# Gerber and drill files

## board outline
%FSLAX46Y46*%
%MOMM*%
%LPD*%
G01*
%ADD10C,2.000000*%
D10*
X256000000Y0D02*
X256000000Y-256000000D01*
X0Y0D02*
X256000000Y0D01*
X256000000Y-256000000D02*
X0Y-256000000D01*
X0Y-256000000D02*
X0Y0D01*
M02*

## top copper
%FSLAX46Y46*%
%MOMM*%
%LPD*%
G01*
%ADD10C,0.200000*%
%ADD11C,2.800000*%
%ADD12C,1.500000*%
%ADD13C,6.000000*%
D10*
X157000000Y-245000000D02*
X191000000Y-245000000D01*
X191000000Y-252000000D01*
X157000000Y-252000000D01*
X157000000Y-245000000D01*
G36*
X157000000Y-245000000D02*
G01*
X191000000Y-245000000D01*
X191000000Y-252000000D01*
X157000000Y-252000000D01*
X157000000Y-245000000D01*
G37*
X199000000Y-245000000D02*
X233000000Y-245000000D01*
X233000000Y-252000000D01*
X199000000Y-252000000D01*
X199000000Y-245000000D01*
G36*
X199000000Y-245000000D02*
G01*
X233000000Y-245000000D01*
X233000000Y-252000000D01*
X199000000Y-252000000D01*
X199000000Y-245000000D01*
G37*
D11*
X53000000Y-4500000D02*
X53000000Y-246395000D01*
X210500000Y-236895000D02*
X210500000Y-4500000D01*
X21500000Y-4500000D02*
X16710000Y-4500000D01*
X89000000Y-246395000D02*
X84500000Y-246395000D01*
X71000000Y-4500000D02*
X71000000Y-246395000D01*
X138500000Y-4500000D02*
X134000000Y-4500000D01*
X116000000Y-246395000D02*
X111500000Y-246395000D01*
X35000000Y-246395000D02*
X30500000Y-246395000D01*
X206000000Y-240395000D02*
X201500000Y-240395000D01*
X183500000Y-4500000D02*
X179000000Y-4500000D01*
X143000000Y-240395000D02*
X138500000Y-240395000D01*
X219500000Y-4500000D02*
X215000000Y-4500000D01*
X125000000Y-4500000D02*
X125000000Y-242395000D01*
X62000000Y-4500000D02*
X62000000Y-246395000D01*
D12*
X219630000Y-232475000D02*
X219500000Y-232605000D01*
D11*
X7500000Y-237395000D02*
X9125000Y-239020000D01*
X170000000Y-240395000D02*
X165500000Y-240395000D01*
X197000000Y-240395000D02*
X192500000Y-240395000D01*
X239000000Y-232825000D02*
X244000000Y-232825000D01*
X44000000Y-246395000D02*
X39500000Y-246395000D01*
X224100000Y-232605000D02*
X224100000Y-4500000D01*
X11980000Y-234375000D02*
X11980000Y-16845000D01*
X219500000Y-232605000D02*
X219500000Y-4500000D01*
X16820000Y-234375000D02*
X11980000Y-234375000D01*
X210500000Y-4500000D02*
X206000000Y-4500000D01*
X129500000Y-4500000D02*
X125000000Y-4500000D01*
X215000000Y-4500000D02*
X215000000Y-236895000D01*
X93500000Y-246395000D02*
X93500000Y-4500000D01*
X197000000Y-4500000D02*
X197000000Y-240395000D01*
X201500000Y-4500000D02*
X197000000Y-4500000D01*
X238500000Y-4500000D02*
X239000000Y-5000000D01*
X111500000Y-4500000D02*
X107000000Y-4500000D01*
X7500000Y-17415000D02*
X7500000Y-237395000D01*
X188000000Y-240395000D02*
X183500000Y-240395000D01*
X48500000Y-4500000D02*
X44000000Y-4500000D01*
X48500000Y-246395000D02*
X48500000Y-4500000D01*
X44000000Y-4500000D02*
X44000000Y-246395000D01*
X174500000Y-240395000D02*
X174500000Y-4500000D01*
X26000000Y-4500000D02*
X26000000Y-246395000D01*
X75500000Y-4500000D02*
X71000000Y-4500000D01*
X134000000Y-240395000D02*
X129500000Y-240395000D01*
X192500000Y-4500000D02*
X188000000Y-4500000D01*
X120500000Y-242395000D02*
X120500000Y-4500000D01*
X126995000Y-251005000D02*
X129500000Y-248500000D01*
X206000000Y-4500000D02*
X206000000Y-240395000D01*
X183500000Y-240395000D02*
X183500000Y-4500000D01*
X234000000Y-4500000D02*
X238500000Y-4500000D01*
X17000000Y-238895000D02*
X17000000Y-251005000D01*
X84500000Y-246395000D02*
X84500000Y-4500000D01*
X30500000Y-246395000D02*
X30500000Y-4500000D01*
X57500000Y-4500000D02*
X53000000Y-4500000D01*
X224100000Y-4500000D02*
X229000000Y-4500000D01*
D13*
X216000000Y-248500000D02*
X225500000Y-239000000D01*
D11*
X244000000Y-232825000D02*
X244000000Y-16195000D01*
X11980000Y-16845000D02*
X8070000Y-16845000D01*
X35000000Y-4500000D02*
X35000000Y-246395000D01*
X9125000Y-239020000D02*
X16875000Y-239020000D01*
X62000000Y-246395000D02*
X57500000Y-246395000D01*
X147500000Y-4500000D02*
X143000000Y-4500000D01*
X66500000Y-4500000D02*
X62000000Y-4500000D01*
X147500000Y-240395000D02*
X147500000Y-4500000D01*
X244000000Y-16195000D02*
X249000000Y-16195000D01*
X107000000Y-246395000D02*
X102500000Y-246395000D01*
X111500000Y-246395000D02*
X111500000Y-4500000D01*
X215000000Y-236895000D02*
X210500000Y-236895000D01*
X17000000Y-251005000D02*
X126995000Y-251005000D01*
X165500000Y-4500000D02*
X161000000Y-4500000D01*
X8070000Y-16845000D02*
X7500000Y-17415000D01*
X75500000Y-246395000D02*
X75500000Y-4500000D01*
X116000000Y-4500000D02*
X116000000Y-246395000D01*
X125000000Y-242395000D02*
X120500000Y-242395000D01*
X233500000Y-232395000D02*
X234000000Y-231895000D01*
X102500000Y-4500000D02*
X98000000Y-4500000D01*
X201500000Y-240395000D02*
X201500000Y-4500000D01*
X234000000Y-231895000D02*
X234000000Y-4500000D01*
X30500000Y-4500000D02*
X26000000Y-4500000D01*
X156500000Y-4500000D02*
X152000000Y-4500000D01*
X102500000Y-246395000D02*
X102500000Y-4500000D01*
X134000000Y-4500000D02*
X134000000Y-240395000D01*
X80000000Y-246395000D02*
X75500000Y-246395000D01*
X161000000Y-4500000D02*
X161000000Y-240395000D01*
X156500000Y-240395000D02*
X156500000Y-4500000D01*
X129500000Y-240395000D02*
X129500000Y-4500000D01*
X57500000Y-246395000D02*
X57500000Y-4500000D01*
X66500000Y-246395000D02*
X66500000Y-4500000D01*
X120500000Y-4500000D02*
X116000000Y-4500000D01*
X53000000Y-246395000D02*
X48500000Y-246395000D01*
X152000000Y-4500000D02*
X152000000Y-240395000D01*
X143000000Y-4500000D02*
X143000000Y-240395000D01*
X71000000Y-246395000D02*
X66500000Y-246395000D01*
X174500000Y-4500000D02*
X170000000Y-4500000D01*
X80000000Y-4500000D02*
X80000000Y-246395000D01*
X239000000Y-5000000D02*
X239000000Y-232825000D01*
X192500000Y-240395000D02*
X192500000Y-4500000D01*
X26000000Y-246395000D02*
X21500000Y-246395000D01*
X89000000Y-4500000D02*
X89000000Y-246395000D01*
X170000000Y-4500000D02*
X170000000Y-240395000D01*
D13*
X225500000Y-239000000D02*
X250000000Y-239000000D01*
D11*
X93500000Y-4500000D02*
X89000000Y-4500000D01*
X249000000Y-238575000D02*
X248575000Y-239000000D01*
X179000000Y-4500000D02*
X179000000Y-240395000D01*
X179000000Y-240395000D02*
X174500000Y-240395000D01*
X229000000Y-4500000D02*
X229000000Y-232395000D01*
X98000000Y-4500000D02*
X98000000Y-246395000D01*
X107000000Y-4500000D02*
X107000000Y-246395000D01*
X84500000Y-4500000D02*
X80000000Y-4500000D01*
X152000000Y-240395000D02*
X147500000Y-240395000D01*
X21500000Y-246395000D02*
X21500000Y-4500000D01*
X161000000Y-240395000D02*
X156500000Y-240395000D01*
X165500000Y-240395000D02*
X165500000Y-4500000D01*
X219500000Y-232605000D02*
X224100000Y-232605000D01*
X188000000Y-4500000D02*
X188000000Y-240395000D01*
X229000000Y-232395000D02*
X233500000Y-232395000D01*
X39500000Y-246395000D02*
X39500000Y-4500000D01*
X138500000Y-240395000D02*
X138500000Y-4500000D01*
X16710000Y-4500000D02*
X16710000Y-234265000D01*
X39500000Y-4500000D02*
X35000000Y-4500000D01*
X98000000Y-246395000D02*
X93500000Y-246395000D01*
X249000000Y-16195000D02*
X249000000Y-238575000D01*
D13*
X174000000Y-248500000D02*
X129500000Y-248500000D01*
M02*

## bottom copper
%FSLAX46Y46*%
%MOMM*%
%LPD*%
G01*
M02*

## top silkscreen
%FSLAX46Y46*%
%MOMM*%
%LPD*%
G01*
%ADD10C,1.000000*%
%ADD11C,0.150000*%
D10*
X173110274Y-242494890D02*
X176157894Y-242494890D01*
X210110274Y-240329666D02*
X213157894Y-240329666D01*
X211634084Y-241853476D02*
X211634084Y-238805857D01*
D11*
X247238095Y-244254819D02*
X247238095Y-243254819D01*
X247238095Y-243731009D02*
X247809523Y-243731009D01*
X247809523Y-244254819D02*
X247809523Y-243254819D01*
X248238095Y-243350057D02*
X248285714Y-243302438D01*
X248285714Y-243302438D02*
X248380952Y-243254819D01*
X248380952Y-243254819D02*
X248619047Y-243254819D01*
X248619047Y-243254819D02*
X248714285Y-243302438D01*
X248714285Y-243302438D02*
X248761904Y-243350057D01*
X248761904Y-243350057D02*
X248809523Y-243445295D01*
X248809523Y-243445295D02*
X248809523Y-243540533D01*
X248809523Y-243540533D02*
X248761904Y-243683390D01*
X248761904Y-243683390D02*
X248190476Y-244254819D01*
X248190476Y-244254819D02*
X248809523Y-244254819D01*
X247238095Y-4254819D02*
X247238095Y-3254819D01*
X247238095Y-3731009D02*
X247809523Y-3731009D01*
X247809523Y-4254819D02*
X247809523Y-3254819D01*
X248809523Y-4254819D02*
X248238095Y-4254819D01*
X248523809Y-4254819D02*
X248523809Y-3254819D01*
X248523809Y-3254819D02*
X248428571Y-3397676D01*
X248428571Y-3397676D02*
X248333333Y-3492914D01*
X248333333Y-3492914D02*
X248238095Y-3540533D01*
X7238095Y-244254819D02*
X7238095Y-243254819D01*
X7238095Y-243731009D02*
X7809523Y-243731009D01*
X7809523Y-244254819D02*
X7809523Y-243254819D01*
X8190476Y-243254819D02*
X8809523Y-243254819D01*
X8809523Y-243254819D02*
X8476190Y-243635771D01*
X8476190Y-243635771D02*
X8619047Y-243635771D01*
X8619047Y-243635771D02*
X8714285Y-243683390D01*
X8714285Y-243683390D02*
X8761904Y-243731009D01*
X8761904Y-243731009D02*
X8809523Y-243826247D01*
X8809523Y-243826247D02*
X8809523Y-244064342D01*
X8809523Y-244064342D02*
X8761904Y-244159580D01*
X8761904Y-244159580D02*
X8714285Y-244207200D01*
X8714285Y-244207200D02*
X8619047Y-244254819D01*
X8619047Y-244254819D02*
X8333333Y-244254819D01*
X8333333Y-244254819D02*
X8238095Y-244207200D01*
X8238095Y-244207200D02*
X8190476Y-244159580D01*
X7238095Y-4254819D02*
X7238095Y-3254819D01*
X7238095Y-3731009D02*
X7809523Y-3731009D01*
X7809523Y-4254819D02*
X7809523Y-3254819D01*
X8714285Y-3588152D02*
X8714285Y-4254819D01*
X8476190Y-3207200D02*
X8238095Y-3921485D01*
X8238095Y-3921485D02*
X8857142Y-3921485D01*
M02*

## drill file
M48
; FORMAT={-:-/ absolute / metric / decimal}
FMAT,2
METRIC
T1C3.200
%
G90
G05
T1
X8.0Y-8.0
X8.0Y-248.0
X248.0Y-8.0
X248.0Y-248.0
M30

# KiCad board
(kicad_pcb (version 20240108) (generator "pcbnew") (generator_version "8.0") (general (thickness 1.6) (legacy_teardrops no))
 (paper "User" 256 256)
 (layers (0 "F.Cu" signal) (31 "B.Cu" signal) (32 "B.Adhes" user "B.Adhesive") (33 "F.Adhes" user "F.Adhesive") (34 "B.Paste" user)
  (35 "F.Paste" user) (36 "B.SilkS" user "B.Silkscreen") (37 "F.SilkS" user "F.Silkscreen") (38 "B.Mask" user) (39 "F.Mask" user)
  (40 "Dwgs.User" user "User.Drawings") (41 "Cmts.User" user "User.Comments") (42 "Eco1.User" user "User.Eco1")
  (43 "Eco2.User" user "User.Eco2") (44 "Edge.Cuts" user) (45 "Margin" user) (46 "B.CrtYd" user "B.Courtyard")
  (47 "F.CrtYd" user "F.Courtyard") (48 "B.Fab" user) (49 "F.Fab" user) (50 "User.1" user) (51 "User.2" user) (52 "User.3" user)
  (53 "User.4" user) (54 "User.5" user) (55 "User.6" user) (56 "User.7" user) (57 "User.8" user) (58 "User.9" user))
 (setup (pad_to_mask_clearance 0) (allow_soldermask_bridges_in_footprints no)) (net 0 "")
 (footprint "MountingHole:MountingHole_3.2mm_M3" (layer "F.Cu") (at 248 248)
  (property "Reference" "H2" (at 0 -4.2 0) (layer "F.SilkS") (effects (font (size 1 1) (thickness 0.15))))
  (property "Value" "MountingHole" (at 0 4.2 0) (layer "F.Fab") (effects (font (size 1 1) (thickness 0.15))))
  (pad "" np_thru_hole circle (at 0 0) (size 3.2 3.2) (drill 3.2) (layers "*.Cu" "*.Mask")))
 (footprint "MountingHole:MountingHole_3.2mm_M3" (layer "F.Cu") (at 248 8)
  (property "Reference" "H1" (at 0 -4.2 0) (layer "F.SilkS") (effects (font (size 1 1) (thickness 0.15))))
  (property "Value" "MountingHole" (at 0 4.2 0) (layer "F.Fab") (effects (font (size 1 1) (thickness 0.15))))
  (pad "" np_thru_hole circle (at 0 0) (size 3.2 3.2) (drill 3.2) (layers "*.Cu" "*.Mask")))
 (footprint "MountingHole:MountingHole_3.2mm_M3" (layer "F.Cu") (at 8 248)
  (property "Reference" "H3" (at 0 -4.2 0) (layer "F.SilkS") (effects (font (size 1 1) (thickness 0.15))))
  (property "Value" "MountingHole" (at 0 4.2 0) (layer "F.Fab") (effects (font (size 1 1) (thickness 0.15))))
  (pad "" np_thru_hole circle (at 0 0) (size 3.2 3.2) (drill 3.2) (layers "*.Cu" "*.Mask")))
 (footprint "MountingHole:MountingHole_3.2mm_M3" (layer "F.Cu") (at 8 8)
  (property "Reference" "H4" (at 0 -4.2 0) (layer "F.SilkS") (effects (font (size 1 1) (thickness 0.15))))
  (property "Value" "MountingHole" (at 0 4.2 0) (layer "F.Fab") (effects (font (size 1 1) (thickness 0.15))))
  (pad "" np_thru_hole circle (at 0 0) (size 3.2 3.2) (drill 3.2) (layers "*.Cu" "*.Mask")))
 (gr_rect (start 157 245) (end 191 252) (stroke (width 0.2) (type solid)) (fill solid) (layer "F.Cu"))
 (gr_rect (start 199 245) (end 233 252) (stroke (width 0.2) (type solid)) (fill solid) (layer "F.Cu"))
 (gr_line (start 256 0) (end 256 256) (stroke (width 2) (type default)) (layer "Edge.Cuts"))
 (gr_line (start 0 0) (end 256 0) (stroke (width 2) (type default)) (layer "Edge.Cuts"))
 (gr_line (start 256 256) (end 0 256) (stroke (width 2) (type default)) (layer "Edge.Cuts"))
 (gr_line (start 0 256) (end 0 0) (stroke (width 2) (type default)) (layer "Edge.Cuts"))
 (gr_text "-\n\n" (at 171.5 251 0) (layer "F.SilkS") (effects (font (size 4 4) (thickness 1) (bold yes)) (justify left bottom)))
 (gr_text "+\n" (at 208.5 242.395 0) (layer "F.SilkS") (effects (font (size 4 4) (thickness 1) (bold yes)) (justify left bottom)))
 (segment (start 53 4.5) (end 53 246.395) (width 2.8) (layer "F.Cu") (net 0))
 (segment (start 210.5 236.895) (end 210.5 4.5) (width 2.8) (layer "F.Cu") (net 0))
 (segment (start 21.5 4.5) (end 16.71 4.5) (width 2.8) (layer "F.Cu") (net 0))
 (segment (start 89 246.395) (end 84.5 246.395) (width 2.8) (layer "F.Cu") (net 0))
 (segment (start 71 4.5) (end 71 246.395) (width 2.8) (layer "F.Cu") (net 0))
 (segment (start 138.5 4.5) (end 134 4.5) (width 2.8) (layer "F.Cu") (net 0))
 (segment (start 116 246.395) (end 111.5 246.395) (width 2.8) (layer "F.Cu") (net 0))
 (segment (start 35 246.395) (end 30.5 246.395) (width 2.8) (layer "F.Cu") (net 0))
 (segment (start 206 240.395) (end 201.5 240.395) (width 2.8) (layer "F.Cu") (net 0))
 (segment (start 183.5 4.5) (end 179 4.5) (width 2.8) (layer "F.Cu") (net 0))
 (segment (start 143 240.395) (end 138.5 240.395) (width 2.8) (layer "F.Cu") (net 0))
 (segment (start 219.5 4.5) (end 215 4.5) (width 2.8) (layer "F.Cu") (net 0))
 (segment (start 125 4.5) (end 125 242.395) (width 2.8) (layer "F.Cu") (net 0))
 (segment (start 62 4.5) (end 62 246.395) (width 2.8) (layer "F.Cu") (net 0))
 (segment (start 219.63 232.475) (end 219.5 232.605) (width 1.5) (layer "F.Cu") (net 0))
 (segment (start 7.5 237.395) (end 9.125 239.02) (width 2.8) (layer "F.Cu") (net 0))
 (segment (start 170 240.395) (end 165.5 240.395) (width 2.8) (layer "F.Cu") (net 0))
 (segment (start 197 240.395) (end 192.5 240.395) (width 2.8) (layer "F.Cu") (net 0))
 (segment (start 239 232.825) (end 244 232.825) (width 2.8) (layer "F.Cu") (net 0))
 (segment (start 44 246.395) (end 39.5 246.395) (width 2.8) (layer "F.Cu") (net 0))
 (segment (start 224.1 232.605) (end 224.1 4.5) (width 2.8) (layer "F.Cu") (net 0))
 (segment (start 11.98 234.375) (end 11.98 16.845) (width 2.8) (layer "F.Cu") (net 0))
 (segment (start 219.5 232.605) (end 219.5 4.5) (width 2.8) (layer "F.Cu") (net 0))
 (segment (start 16.82 234.375) (end 11.98 234.375) (width 2.8) (layer "F.Cu") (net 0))
 (segment (start 210.5 4.5) (end 206 4.5) (width 2.8) (layer "F.Cu") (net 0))
 (segment (start 129.5 4.5) (end 125 4.5) (width 2.8) (layer "F.Cu") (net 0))
 (segment (start 215 4.5) (end 215 236.895) (width 2.8) (layer "F.Cu") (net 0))
 (segment (start 93.5 246.395) (end 93.5 4.5) (width 2.8) (layer "F.Cu") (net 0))
 (segment (start 197 4.5) (end 197 240.395) (width 2.8) (layer "F.Cu") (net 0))
 (segment (start 201.5 4.5) (end 197 4.5) (width 2.8) (layer "F.Cu") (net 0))
 (segment (start 238.5 4.5) (end 239 5) (width 2.8) (layer "F.Cu") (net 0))
 (segment (start 111.5 4.5) (end 107 4.5) (width 2.8) (layer "F.Cu") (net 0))
 (segment (start 7.5 17.415) (end 7.5 237.395) (width 2.8) (layer "F.Cu") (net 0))
 (segment (start 188 240.395) (end 183.5 240.395) (width 2.8) (layer "F.Cu") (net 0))
 (segment (start 48.5 4.5) (end 44 4.5) (width 2.8) (layer "F.Cu") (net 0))
 (segment (start 48.5 246.395) (end 48.5 4.5) (width 2.8) (layer "F.Cu") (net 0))
 (segment (start 44 4.5) (end 44 246.395) (width 2.8) (layer "F.Cu") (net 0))
 (segment (start 174.5 240.395) (end 174.5 4.5) (width 2.8) (layer "F.Cu") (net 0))
 (segment (start 26 4.5) (end 26 246.395) (width 2.8) (layer "F.Cu") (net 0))
 (segment (start 75.5 4.5) (end 71 4.5) (width 2.8) (layer "F.Cu") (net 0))
 (segment (start 134 240.395) (end 129.5 240.395) (width 2.8) (layer "F.Cu") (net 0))
 (segment (start 192.5 4.5) (end 188 4.5) (width 2.8) (layer "F.Cu") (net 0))
 (segment (start 120.5 242.395) (end 120.5 4.5) (width 2.8) (layer "F.Cu") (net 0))
 (segment (start 126.995 251.005) (end 129.5 248.5) (width 2.8) (layer "F.Cu") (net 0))
 (segment (start 206 4.5) (end 206 240.395) (width 2.8) (layer "F.Cu") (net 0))
 (segment (start 183.5 240.395) (end 183.5 4.5) (width 2.8) (layer "F.Cu") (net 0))
 (segment (start 234 4.5) (end 238.5 4.5) (width 2.8) (layer "F.Cu") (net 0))
 (segment (start 17 238.895) (end 17 251.005) (width 2.8) (layer "F.Cu") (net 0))
 (segment (start 84.5 246.395) (end 84.5 4.5) (width 2.8) (layer "F.Cu") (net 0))
 (segment (start 30.5 246.395) (end 30.5 4.5) (width 2.8) (layer "F.Cu") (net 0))
 (segment (start 57.5 4.5) (end 53 4.5) (width 2.8) (layer "F.Cu") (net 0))
 (segment (start 224.1 4.5) (end 229 4.5) (width 2.8) (layer "F.Cu") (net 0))
 (segment (start 216 248.5) (end 225.5 239) (width 6) (layer "F.Cu") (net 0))
 (segment (start 244 232.825) (end 244 16.195) (width 2.8) (layer "F.Cu") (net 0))
 (segment (start 11.98 16.845) (end 8.07 16.845) (width 2.8) (layer "F.Cu") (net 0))
 (segment (start 35 4.5) (end 35 246.395) (width 2.8) (layer "F.Cu") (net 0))
 (segment (start 9.125 239.02) (end 16.875 239.02) (width 2.8) (layer "F.Cu") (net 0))
 (segment (start 62 246.395) (end 57.5 246.395) (width 2.8) (layer "F.Cu") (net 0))
 (segment (start 147.5 4.5) (end 143 4.5) (width 2.8) (layer "F.Cu") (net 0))
 (segment (start 66.5 4.5) (end 62 4.5) (width 2.8) (layer "F.Cu") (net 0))
 (segment (start 147.5 240.395) (end 147.5 4.5) (width 2.8) (layer "F.Cu") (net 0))
 (segment (start 244 16.195) (end 249 16.195) (width 2.8) (layer "F.Cu") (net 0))
 (segment (start 107 246.395) (end 102.5 246.395) (width 2.8) (layer "F.Cu") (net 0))
 (segment (start 111.5 246.395) (end 111.5 4.5) (width 2.8) (layer "F.Cu") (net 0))
 (segment (start 215 236.895) (end 210.5 236.895) (width 2.8) (layer "F.Cu") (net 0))
 (segment (start 17 251.005) (end 126.995 251.005) (width 2.8) (layer "F.Cu") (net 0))
 (segment (start 165.5 4.5) (end 161 4.5) (width 2.8) (layer "F.Cu") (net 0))
 (segment (start 8.07 16.845) (end 7.5 17.415) (width 2.8) (layer "F.Cu") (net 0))
 (segment (start 75.5 246.395) (end 75.5 4.5) (width 2.8) (layer "F.Cu") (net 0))
 (segment (start 116 4.5) (end 116 246.395) (width 2.8) (layer "F.Cu") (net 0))
 (segment (start 125 242.395) (end 120.5 242.395) (width 2.8) (layer "F.Cu") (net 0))
 (segment (start 233.5 232.395) (end 234 231.895) (width 2.8) (layer "F.Cu") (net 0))
 (segment (start 102.5 4.5) (end 98 4.5) (width 2.8) (layer "F.Cu") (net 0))
 (segment (start 201.5 240.395) (end 201.5 4.5) (width 2.8) (layer "F.Cu") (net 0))
 (segment (start 234 231.895) (end 234 4.5) (width 2.8) (layer "F.Cu") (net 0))
 (segment (start 30.5 4.5) (end 26 4.5) (width 2.8) (layer "F.Cu") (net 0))
 (segment (start 156.5 4.5) (end 152 4.5) (width 2.8) (layer "F.Cu") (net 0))
 (segment (start 102.5 246.395) (end 102.5 4.5) (width 2.8) (layer "F.Cu") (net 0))
 (segment (start 134 4.5) (end 134 240.395) (width 2.8) (layer "F.Cu") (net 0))
 (segment (start 80 246.395) (end 75.5 246.395) (width 2.8) (layer "F.Cu") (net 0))
 (segment (start 161 4.5) (end 161 240.395) (width 2.8) (layer "F.Cu") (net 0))
 (segment (start 156.5 240.395) (end 156.5 4.5) (width 2.8) (layer "F.Cu") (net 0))
 (segment (start 129.5 240.395) (end 129.5 4.5) (width 2.8) (layer "F.Cu") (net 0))
 (segment (start 57.5 246.395) (end 57.5 4.5) (width 2.8) (layer "F.Cu") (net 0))
 (segment (start 66.5 246.395) (end 66.5 4.5) (width 2.8) (layer "F.Cu") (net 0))
 (segment (start 120.5 4.5) (end 116 4.5) (width 2.8) (layer "F.Cu") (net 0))
 (segment (start 53 246.395) (end 48.5 246.395) (width 2.8) (layer "F.Cu") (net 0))
 (segment (start 152 4.5) (end 152 240.395) (width 2.8) (layer "F.Cu") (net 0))
 (segment (start 143 4.5) (end 143 240.395) (width 2.8) (layer "F.Cu") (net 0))
 (segment (start 71 246.395) (end 66.5 246.395) (width 2.8) (layer "F.Cu") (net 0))
 (segment (start 174.5 4.5) (end 170 4.5) (width 2.8) (layer "F.Cu") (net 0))
 (segment (start 80 4.5) (end 80 246.395) (width 2.8) (layer "F.Cu") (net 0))
 (segment (start 239 5) (end 239 232.825) (width 2.8) (layer "F.Cu") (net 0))
 (segment (start 192.5 240.395) (end 192.5 4.5) (width 2.8) (layer "F.Cu") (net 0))
 (segment (start 26 246.395) (end 21.5 246.395) (width 2.8) (layer "F.Cu") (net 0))
 (segment (start 89 4.5) (end 89 246.395) (width 2.8) (layer "F.Cu") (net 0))
 (segment (start 170 4.5) (end 170 240.395) (width 2.8) (layer "F.Cu") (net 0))
 (segment (start 225.5 239) (end 250 239) (width 6) (layer "F.Cu") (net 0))
 (segment (start 93.5 4.5) (end 89 4.5) (width 2.8) (layer "F.Cu") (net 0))
 (segment (start 249 238.575) (end 248.575 239) (width 2.8) (layer "F.Cu") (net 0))
 (segment (start 179 4.5) (end 179 240.395) (width 2.8) (layer "F.Cu") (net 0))
 (segment (start 179 240.395) (end 174.5 240.395) (width 2.8) (layer "F.Cu") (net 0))
 (segment (start 229 4.5) (end 229 232.395) (width 2.8) (layer "F.Cu") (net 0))
 (segment (start 98 4.5) (end 98 246.395) (width 2.8) (layer "F.Cu") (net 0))
 (segment (start 107 4.5) (end 107 246.395) (width 2.8) (layer "F.Cu") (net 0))
 (segment (start 84.5 4.5) (end 80 4.5) (width 2.8) (layer "F.Cu") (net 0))
 (segment (start 152 240.395) (end 147.5 240.395) (width 2.8) (layer "F.Cu") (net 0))
 (segment (start 21.5 246.395) (end 21.5 4.5) (width 2.8) (layer "F.Cu") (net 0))
 (segment (start 161 240.395) (end 156.5 240.395) (width 2.8) (layer "F.Cu") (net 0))
 (segment (start 165.5 240.395) (end 165.5 4.5) (width 2.8) (layer "F.Cu") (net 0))
 (segment (start 219.5 232.605) (end 224.1 232.605) (width 2.8) (layer "F.Cu") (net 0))
 (segment (start 188 4.5) (end 188 240.395) (width 2.8) (layer "F.Cu") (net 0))
 (segment (start 229 232.395) (end 233.5 232.395) (width 2.8) (layer "F.Cu") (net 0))
 (segment (start 39.5 246.395) (end 39.5 4.5) (width 2.8) (layer "F.Cu") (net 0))
 (segment (start 138.5 240.395) (end 138.5 4.5) (width 2.8) (layer "F.Cu") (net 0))
 (segment (start 16.71 4.5) (end 16.71 234.265) (width 2.8) (layer "F.Cu") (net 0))
 (segment (start 39.5 4.5) (end 35 4.5) (width 2.8) (layer "F.Cu") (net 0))
 (segment (start 98 246.395) (end 93.5 246.395) (width 2.8) (layer "F.Cu") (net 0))
 (segment (start 249 16.195) (end 249 238.575) (width 2.8) (layer "F.Cu") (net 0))
 (segment (start 174 248.5) (end 129.5 248.5) (width 6) (layer "F.Cu") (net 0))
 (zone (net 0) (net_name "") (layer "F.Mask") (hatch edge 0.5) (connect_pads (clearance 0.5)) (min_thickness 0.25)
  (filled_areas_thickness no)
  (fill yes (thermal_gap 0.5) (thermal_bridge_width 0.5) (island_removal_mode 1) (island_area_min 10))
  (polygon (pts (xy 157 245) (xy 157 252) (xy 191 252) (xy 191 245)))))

